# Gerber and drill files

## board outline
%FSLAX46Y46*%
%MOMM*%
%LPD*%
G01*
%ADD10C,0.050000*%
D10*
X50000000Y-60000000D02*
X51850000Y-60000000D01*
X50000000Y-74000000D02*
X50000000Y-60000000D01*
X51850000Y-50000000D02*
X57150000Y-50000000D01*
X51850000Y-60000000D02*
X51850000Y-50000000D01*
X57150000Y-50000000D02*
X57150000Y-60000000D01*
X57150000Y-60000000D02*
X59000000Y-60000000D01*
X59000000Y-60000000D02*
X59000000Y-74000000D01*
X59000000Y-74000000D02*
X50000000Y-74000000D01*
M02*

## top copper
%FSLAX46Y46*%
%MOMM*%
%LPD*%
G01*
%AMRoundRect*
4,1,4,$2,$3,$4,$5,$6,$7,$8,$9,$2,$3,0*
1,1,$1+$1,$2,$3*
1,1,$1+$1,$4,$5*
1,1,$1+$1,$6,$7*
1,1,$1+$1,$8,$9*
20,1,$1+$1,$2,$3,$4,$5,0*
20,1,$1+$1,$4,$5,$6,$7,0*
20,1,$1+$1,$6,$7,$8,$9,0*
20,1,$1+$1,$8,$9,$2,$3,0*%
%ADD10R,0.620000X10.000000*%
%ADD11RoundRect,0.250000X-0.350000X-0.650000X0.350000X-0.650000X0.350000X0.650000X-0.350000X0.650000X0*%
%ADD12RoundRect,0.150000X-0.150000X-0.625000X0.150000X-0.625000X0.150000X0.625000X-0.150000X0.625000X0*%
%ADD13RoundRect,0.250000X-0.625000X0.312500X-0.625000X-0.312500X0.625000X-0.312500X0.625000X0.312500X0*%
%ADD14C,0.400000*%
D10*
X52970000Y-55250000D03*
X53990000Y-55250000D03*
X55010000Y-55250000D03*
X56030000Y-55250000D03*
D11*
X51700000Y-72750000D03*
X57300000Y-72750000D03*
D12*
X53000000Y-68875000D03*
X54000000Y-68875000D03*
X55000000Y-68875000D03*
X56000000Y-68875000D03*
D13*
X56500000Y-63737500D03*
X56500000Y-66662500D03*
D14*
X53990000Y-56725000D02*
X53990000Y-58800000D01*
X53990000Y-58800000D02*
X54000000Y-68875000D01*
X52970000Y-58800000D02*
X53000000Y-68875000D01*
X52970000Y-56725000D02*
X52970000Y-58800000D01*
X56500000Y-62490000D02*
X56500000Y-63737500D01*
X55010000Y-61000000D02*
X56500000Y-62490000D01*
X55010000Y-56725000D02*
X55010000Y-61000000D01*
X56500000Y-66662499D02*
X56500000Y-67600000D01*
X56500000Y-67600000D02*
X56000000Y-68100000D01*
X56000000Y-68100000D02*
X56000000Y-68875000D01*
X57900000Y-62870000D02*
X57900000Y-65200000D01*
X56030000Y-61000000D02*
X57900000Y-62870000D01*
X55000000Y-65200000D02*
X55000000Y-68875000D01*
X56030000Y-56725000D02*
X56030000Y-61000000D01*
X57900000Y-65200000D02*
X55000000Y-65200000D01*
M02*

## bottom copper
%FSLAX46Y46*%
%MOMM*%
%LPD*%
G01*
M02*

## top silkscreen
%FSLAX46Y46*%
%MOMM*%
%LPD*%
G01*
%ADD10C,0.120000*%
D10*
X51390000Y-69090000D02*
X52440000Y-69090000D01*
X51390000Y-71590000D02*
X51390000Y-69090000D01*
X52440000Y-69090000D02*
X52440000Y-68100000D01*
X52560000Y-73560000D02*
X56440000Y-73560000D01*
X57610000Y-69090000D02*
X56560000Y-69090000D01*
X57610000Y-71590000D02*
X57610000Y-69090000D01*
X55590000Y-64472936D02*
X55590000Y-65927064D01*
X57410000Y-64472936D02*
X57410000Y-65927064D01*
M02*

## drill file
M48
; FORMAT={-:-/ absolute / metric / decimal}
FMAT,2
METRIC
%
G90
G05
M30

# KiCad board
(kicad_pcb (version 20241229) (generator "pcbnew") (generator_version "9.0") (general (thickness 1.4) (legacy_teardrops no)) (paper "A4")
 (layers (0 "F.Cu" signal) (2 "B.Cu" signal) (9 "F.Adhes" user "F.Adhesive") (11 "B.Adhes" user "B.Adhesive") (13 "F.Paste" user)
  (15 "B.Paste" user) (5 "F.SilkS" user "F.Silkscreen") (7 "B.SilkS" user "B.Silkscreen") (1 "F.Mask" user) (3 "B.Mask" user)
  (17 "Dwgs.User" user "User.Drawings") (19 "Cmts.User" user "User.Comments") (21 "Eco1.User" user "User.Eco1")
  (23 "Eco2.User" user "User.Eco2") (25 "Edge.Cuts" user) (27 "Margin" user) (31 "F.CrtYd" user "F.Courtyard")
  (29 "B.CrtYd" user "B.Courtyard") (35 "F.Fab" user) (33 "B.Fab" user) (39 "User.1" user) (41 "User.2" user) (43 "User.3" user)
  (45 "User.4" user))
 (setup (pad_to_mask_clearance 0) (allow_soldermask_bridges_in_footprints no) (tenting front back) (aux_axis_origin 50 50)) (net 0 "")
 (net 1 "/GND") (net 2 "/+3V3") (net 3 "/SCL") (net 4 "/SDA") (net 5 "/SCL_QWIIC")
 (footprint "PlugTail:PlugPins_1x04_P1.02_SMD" (layer "F.Cu") (at 54.5 50)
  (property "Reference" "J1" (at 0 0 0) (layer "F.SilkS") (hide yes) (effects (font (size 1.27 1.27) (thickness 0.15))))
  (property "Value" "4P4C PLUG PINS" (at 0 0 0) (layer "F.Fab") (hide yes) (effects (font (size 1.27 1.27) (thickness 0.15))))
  (pad "1" smd rect (at -1.53 5.25) (size 0.62 10) (layers "F.Cu" "F.Mask") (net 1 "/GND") (thermal_bridge_angle 45))
  (pad "2" smd rect (at -0.51 5.25) (size 0.62 10) (layers "F.Cu" "F.Mask") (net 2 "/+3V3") (thermal_bridge_angle 45))
  (pad "3" smd rect (at 0.51 5.25) (size 0.62 10) (layers "F.Cu" "F.Mask") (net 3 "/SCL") (thermal_bridge_angle 45))
  (pad "4" smd rect (at 1.53 5.25) (size 0.62 10) (layers "F.Cu" "F.Mask") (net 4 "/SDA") (thermal_bridge_angle 45)))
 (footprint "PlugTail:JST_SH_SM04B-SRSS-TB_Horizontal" (layer "F.Cu") (at 54.5 70.875)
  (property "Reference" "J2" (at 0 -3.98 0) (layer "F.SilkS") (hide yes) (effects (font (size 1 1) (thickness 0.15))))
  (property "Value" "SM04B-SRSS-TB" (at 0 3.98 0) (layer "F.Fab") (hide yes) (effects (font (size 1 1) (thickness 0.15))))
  (fp_line (start -3.11 -1.785) (end -2.06 -1.785) (stroke (width 0.12) (type solid)) (layer "F.SilkS"))
  (fp_line (start -3.11 0.715) (end -3.11 -1.785) (stroke (width 0.12) (type solid)) (layer "F.SilkS"))
  (fp_line (start -2.06 -1.785) (end -2.06 -2.775) (stroke (width 0.12) (type solid)) (layer "F.SilkS"))
  (fp_line (start -1.94 2.685) (end 1.94 2.685) (stroke (width 0.12) (type solid)) (layer "F.SilkS"))
  (fp_line (start 3.11 -1.785) (end 2.06 -1.785) (stroke (width 0.12) (type solid)) (layer "F.SilkS"))
  (fp_line (start 3.11 0.715) (end 3.11 -1.785) (stroke (width 0.12) (type solid)) (layer "F.SilkS"))
  (pad "" smd roundrect (at -2.8 1.875) (size 1.2 1.8) (layers "F.Cu" "F.Mask" "F.Paste") (roundrect_rratio 0.208333))
  (pad "" smd roundrect (at 2.8 1.875) (size 1.2 1.8) (layers "F.Cu" "F.Mask" "F.Paste") (roundrect_rratio 0.208333))
  (pad "1" smd roundrect (at -1.5 -2) (size 0.6 1.55) (layers "F.Cu" "F.Mask" "F.Paste") (roundrect_rratio 0.25) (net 1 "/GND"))
  (pad "2" smd roundrect (at -0.5 -2) (size 0.6 1.55) (layers "F.Cu" "F.Mask" "F.Paste") (roundrect_rratio 0.25) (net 2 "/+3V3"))
  (pad "3" smd roundrect (at 0.5 -2) (size 0.6 1.55) (layers "F.Cu" "F.Mask" "F.Paste") (roundrect_rratio 0.25) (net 4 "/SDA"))
  (pad "4" smd roundrect (at 1.5 -2) (size 0.6 1.55) (layers "F.Cu" "F.Mask" "F.Paste") (roundrect_rratio 0.25) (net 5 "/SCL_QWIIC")))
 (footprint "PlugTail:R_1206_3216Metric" (layer "F.Cu") (at 56.5 65.2 -90)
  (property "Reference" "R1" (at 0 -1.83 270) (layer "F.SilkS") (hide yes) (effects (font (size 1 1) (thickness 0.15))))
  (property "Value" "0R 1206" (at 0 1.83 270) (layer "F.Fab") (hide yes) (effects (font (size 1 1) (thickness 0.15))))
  (fp_line (start -0.727064 0.91) (end 0.727064 0.91) (stroke (width 0.12) (type solid)) (layer "F.SilkS"))
  (fp_line (start -0.727064 -0.91) (end 0.727064 -0.91) (stroke (width 0.12) (type solid)) (layer "F.SilkS"))
  (pad "1" smd roundrect (at -1.4625 0 270) (size 1.125 1.75) (layers "F.Cu" "F.Mask" "F.Paste") (roundrect_rratio 0.222222) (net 3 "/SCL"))
  (pad "2" smd roundrect (at 1.4625 0 270) (size 1.125 1.75) (layers "F.Cu" "F.Mask" "F.Paste") (roundrect_rratio 0.222222)
   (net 5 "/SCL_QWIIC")))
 (gr_line (start 50 60) (end 51.85 60) (stroke (width 0.05) (type default)) (layer "Edge.Cuts"))
 (gr_line (start 50 74) (end 50 60) (stroke (width 0.05) (type default)) (layer "Edge.Cuts"))
 (gr_line (start 51.85 50) (end 57.15 50) (stroke (width 0.05) (type default)) (layer "Edge.Cuts"))
 (gr_line (start 51.85 60) (end 51.85 50) (stroke (width 0.05) (type default)) (layer "Edge.Cuts"))
 (gr_line (start 57.15 50) (end 57.15 60) (stroke (width 0.05) (type default)) (layer "Edge.Cuts"))
 (gr_line (start 57.15 60) (end 59 60) (stroke (width 0.05) (type default)) (layer "Edge.Cuts"))
 (gr_line (start 59 60) (end 59 74) (stroke (width 0.05) (type default)) (layer "Edge.Cuts"))
 (gr_line (start 59 74) (end 50 74) (stroke (width 0.05) (type default)) (layer "Edge.Cuts"))
 (segment (start 53.99 56.725) (end 53.99 58.8) (width 0.4) (layer "F.Cu") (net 2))
 (segment (start 53.99 58.8) (end 54 68.875) (width 0.4) (layer "F.Cu") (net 2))
 (segment (start 52.97 58.8) (end 53 68.875) (width 0.4) (layer "F.Cu") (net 1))
 (segment (start 52.97 56.725) (end 52.97 58.8) (width 0.4) (layer "F.Cu") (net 1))
 (segment (start 56.5 62.49) (end 56.5 63.7375) (width 0.4) (layer "F.Cu") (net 3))
 (segment (start 55.01 61) (end 56.5 62.49) (width 0.4) (layer "F.Cu") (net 3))
 (segment (start 55.01 56.725) (end 55.01 61) (width 0.4) (layer "F.Cu") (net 3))
 (segment (start 56.5 66.662499) (end 56.5 67.6) (width 0.4) (layer "F.Cu") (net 5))
 (segment (start 56.5 67.6) (end 56 68.1) (width 0.4) (layer "F.Cu") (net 5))
 (segment (start 56 68.1) (end 56 68.875) (width 0.4) (layer "F.Cu") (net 5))
 (segment (start 57.9 62.87) (end 57.9 65.2) (width 0.4) (layer "F.Cu") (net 4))
 (segment (start 56.03 61) (end 57.9 62.87) (width 0.4) (layer "F.Cu") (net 4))
 (segment (start 55 65.2) (end 55 68.875) (width 0.4) (layer "F.Cu") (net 4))
 (segment (start 56.03 56.725) (end 56.03 61) (width 0.4) (layer "F.Cu") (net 4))
 (segment (start 57.9 65.2) (end 55 65.2) (width 0.4) (layer "F.Cu") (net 4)))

